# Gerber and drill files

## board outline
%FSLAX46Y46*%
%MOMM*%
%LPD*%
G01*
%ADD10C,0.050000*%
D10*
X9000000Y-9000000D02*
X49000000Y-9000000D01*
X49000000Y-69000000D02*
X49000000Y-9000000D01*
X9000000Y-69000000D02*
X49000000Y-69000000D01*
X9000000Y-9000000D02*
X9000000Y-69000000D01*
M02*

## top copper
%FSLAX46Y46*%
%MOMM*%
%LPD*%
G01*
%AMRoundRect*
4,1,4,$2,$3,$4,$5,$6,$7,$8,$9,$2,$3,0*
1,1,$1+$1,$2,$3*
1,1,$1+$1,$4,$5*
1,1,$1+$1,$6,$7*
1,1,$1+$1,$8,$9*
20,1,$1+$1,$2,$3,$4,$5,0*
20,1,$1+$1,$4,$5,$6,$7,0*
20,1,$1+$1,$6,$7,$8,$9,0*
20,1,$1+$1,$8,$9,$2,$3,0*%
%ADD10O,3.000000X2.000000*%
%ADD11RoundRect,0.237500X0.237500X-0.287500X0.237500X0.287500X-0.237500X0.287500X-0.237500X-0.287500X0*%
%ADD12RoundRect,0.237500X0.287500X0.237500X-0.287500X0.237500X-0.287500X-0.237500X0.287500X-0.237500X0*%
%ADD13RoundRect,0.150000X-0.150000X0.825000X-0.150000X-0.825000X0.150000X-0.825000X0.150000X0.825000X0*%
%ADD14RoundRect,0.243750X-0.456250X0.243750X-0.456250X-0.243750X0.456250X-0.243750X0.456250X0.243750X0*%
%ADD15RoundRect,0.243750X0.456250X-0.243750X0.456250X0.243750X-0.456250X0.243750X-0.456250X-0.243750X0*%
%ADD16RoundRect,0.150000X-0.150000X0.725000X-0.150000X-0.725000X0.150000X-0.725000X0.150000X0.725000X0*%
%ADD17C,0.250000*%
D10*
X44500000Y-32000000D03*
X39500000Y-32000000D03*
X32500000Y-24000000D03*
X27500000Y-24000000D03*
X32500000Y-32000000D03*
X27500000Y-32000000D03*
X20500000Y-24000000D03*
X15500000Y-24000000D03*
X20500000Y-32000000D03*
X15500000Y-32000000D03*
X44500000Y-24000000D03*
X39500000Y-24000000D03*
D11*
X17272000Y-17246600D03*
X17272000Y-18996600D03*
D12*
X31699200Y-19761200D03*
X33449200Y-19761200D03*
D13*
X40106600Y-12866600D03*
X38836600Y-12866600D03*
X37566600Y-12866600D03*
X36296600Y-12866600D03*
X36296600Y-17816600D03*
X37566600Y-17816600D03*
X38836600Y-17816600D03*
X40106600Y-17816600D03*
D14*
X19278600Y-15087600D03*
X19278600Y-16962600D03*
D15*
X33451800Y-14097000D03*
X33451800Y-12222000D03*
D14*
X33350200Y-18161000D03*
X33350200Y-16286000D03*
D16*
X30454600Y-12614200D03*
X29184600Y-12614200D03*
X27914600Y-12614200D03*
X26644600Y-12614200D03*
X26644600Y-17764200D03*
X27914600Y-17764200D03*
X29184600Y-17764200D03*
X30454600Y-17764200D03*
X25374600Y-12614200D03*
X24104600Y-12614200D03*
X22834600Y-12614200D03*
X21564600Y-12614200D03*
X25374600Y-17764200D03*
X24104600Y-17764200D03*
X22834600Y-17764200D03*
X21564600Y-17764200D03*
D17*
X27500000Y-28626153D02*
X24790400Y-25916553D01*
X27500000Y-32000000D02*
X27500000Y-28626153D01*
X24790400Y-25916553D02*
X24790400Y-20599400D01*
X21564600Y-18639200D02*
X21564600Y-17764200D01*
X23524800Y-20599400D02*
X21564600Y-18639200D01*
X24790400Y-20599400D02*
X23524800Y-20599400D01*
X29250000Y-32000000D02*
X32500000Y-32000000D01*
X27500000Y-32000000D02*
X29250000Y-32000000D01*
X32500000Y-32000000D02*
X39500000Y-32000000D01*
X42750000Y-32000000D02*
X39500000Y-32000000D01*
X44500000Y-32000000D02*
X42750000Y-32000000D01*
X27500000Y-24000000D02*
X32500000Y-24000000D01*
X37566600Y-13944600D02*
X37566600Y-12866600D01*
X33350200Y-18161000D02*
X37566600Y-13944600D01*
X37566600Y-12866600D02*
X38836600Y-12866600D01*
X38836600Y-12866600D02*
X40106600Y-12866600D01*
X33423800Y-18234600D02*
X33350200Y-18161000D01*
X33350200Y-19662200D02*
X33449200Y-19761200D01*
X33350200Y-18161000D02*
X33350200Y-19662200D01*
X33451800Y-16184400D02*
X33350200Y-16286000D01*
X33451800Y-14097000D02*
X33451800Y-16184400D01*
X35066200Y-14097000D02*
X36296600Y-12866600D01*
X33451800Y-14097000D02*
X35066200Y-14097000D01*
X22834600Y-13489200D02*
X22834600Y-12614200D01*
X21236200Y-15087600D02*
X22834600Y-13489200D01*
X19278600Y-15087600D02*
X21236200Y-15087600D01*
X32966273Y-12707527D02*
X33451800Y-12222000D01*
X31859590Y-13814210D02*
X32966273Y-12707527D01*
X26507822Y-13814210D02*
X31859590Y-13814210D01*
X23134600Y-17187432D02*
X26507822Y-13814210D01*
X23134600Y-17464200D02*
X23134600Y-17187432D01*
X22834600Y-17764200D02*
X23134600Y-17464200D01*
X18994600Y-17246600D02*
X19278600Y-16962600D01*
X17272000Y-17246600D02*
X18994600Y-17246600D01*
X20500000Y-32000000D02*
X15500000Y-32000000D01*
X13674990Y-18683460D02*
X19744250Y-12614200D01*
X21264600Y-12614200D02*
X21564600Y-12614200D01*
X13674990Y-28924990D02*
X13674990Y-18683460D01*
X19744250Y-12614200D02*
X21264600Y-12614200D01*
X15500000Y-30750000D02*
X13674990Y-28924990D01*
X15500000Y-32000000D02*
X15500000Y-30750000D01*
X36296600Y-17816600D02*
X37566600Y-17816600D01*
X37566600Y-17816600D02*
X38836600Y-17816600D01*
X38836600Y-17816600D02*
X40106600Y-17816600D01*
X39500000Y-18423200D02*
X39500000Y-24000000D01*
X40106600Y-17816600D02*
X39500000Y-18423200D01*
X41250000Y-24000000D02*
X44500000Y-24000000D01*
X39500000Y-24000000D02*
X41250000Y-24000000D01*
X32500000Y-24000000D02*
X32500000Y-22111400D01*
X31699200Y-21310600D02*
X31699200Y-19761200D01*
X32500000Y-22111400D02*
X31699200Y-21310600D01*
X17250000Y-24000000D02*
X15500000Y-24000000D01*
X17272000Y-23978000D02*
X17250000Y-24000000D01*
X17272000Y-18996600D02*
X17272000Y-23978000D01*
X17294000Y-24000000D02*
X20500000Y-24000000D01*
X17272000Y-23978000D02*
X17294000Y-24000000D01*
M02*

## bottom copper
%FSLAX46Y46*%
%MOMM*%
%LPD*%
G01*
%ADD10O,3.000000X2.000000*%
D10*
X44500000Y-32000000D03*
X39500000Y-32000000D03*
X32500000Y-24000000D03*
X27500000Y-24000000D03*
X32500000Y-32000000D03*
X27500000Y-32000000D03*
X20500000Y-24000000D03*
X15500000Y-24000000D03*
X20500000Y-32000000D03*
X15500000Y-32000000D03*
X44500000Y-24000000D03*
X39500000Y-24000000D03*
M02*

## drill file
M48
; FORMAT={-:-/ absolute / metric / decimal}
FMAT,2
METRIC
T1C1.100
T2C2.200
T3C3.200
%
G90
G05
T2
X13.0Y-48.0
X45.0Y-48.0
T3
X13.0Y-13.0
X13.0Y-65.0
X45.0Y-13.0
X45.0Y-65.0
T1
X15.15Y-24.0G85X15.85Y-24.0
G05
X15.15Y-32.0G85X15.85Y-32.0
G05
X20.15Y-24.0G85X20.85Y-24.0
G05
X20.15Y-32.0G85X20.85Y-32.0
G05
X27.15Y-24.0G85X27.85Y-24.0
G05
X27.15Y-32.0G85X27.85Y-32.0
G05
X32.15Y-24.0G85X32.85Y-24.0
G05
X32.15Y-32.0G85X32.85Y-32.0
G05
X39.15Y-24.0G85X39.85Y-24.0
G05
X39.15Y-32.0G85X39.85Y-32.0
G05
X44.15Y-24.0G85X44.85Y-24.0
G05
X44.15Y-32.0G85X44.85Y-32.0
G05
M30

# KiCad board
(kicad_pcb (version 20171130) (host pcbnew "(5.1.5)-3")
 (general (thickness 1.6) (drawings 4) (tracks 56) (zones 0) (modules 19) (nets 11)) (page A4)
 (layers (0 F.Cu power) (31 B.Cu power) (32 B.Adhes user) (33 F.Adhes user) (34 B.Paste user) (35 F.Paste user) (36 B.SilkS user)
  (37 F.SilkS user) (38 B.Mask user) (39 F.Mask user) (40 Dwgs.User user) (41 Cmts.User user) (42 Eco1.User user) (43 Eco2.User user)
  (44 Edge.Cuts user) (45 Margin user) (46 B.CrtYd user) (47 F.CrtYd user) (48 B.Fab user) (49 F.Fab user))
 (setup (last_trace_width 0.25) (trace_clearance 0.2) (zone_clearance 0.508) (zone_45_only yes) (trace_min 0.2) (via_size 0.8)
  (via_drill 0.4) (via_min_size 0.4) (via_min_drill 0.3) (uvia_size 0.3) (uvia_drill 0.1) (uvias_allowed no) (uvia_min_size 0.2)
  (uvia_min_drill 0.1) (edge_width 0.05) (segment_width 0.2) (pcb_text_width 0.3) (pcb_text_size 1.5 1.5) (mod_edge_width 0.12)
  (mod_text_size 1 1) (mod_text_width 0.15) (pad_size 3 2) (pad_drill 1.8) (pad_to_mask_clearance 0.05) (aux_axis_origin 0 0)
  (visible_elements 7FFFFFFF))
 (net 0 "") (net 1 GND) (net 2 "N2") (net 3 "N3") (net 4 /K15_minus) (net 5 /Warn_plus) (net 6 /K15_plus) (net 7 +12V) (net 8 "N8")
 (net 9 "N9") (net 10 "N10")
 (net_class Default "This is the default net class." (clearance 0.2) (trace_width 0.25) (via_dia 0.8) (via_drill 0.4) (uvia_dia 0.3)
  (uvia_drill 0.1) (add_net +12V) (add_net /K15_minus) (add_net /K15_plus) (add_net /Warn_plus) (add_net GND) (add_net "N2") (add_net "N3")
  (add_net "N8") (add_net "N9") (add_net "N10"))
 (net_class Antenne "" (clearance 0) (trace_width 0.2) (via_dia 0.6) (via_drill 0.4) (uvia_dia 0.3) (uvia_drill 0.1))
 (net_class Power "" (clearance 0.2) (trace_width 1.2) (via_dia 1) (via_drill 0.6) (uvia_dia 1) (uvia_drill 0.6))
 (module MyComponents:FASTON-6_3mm (layer F.Cu) (at 42 32)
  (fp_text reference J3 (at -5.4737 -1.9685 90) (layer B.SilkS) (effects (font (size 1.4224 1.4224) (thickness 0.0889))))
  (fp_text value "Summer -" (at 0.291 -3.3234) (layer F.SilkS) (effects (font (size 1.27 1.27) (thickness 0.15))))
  (pad 1 thru_hole oval (at 2.5 0) (size 3 2) (drill oval 1.8 1.1) (layers *.Cu *.Paste *.Mask F.SilkS) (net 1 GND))
  (pad 1 thru_hole oval (at -2.5 0) (size 3 2) (drill oval 1.8 1.1) (layers *.Cu *.Paste *.Mask F.SilkS) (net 1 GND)))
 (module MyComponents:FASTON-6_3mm (layer F.Cu) (at 30 24)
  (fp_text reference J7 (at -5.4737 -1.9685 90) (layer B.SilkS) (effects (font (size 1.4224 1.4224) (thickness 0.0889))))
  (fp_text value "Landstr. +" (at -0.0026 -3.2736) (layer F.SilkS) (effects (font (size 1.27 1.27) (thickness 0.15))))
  (pad 1 thru_hole oval (at 2.5 0) (size 3 2) (drill oval 1.8 1.1) (layers *.Cu *.Paste *.Mask F.SilkS) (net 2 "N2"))
  (pad 1 thru_hole oval (at -2.5 0) (size 3 2) (drill oval 1.8 1.1) (layers *.Cu *.Paste *.Mask F.SilkS) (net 2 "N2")))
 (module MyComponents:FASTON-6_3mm (layer F.Cu) (at 30 32)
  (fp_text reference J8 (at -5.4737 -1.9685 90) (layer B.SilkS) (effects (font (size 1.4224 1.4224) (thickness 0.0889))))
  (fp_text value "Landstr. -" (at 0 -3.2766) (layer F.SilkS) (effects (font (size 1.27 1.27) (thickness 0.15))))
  (pad 1 thru_hole oval (at 2.5 0) (size 3 2) (drill oval 1.8 1.1) (layers *.Cu *.Paste *.Mask F.SilkS) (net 1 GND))
  (pad 1 thru_hole oval (at -2.5 0) (size 3 2) (drill oval 1.8 1.1) (layers *.Cu *.Paste *.Mask F.SilkS) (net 1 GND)))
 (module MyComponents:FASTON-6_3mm (layer F.Cu) (at 18 24)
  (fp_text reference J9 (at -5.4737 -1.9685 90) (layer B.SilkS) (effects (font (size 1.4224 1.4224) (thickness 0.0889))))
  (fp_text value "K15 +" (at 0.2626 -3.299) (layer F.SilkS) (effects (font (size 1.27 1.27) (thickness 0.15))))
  (pad 1 thru_hole oval (at 2.5 0) (size 3 2) (drill oval 1.8 1.1) (layers *.Cu *.Paste *.Mask F.SilkS) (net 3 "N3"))
  (pad 1 thru_hole oval (at -2.5 0) (size 3 2) (drill oval 1.8 1.1) (layers *.Cu *.Paste *.Mask F.SilkS) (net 3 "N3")))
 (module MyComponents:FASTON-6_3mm (layer F.Cu) (at 18 32)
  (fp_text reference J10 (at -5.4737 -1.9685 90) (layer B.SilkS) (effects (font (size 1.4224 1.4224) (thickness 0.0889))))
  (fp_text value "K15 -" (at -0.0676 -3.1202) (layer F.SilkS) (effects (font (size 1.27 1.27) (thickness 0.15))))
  (pad 1 thru_hole oval (at 2.5 0) (size 3 2) (drill oval 1.8 1.1) (layers *.Cu *.Paste *.Mask F.SilkS) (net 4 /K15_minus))
  (pad 1 thru_hole oval (at -2.5 0) (size 3 2) (drill oval 1.8 1.1) (layers *.Cu *.Paste *.Mask F.SilkS) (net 4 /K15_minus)))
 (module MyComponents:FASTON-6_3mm (layer F.Cu) (at 42 24)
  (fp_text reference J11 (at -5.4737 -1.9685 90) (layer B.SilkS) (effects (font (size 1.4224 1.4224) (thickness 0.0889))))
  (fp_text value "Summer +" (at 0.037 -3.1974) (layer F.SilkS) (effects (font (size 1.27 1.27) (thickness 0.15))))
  (pad 1 thru_hole oval (at 2.5 0) (size 3 2) (drill oval 1.8 1.1) (layers *.Cu *.Paste *.Mask F.SilkS) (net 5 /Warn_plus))
  (pad 1 thru_hole oval (at -2.5 0) (size 3 2) (drill oval 1.8 1.1) (layers *.Cu *.Paste *.Mask F.SilkS) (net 5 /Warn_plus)))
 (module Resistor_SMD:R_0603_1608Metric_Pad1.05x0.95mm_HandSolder (layer F.Cu) (at 17.272 18.1216 90)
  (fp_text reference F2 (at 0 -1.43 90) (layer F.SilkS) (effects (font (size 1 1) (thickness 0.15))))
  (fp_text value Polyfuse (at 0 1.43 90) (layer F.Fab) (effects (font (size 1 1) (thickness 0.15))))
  (pad 2 smd roundrect (at 0.875 0 90) (size 1.05 0.95) (layers F.Cu F.Paste F.Mask) (roundrect_rratio 0.25) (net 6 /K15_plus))
  (pad 1 smd roundrect (at -0.875 0 90) (size 1.05 0.95) (layers F.Cu F.Paste F.Mask) (roundrect_rratio 0.25) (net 3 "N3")))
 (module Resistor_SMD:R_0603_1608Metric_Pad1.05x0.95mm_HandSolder (layer F.Cu) (at 32.5742 19.7612 180)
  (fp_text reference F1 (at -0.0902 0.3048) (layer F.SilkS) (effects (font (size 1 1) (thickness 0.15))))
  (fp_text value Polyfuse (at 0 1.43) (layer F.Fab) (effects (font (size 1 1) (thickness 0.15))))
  (pad 2 smd roundrect (at 0.875 0 180) (size 1.05 0.95) (layers F.Cu F.Paste F.Mask) (roundrect_rratio 0.25) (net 2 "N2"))
  (pad 1 smd roundrect (at -0.875 0 180) (size 1.05 0.95) (layers F.Cu F.Paste F.Mask) (roundrect_rratio 0.25) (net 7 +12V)))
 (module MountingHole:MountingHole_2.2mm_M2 (layer F.Cu) (at 45 48)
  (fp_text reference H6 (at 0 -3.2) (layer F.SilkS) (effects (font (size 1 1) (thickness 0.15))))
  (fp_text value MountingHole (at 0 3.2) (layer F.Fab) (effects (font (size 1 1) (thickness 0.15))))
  (pad 1 np_thru_hole circle (at 0 0) (size 2.2 2.2) (drill 2.2) (layers *.Cu *.Mask)))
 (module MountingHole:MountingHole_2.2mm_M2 (layer F.Cu) (at 13 48)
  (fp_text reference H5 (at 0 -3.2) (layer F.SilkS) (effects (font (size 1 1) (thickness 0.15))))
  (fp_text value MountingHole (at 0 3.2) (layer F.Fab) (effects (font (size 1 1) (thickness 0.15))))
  (pad 1 np_thru_hole circle (at 0 0) (size 2.2 2.2) (drill 2.2) (layers *.Cu *.Mask)))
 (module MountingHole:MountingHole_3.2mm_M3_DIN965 (layer F.Cu) (at 13 13)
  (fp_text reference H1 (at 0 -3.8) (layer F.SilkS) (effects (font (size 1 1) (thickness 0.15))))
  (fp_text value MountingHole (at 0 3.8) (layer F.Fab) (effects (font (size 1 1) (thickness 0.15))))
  (pad 1 np_thru_hole circle (at 0 0) (size 3.2 3.2) (drill 3.2) (layers *.Cu *.Mask)))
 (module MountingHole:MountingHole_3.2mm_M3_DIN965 (layer F.Cu) (at 13 65)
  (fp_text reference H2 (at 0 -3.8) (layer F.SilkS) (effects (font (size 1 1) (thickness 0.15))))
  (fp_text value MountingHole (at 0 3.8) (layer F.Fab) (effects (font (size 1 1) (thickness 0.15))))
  (pad 1 np_thru_hole circle (at 0 0) (size 3.2 3.2) (drill 3.2) (layers *.Cu *.Mask)))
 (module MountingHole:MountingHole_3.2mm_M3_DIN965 (layer F.Cu) (at 45 13)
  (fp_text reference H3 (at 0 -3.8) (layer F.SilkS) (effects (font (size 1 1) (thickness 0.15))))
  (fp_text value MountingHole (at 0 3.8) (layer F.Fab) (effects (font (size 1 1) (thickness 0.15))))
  (pad 1 np_thru_hole circle (at 0 0) (size 3.2 3.2) (drill 3.2) (layers *.Cu *.Mask)))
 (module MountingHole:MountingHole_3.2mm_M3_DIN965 (layer F.Cu) (at 45 65)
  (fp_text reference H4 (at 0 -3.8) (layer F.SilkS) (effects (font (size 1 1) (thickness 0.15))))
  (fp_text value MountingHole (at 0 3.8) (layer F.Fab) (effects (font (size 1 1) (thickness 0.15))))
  (pad 1 np_thru_hole circle (at 0 0) (size 3.2 3.2) (drill 3.2) (layers *.Cu *.Mask)))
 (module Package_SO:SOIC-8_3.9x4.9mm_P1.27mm (layer F.Cu) (at 38.2016 15.3416 270)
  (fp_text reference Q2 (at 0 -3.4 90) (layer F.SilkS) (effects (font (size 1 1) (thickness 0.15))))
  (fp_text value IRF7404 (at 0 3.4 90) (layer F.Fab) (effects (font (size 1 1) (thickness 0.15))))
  (pad 1 smd roundrect (at -2.475 -1.905 270) (size 1.95 0.6) (layers F.Cu F.Paste F.Mask) (roundrect_rratio 0.25) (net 7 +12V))
  (pad 2 smd roundrect (at -2.475 -0.635 270) (size 1.95 0.6) (layers F.Cu F.Paste F.Mask) (roundrect_rratio 0.25) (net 7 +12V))
  (pad 3 smd roundrect (at -2.475 0.635 270) (size 1.95 0.6) (layers F.Cu F.Paste F.Mask) (roundrect_rratio 0.25) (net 7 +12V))
  (pad 4 smd roundrect (at -2.475 1.905 270) (size 1.95 0.6) (layers F.Cu F.Paste F.Mask) (roundrect_rratio 0.25) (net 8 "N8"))
  (pad 5 smd roundrect (at 2.475 1.905 270) (size 1.95 0.6) (layers F.Cu F.Paste F.Mask) (roundrect_rratio 0.25) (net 5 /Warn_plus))
  (pad 6 smd roundrect (at 2.475 0.635 270) (size 1.95 0.6) (layers F.Cu F.Paste F.Mask) (roundrect_rratio 0.25) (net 5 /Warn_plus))
  (pad 7 smd roundrect (at 2.475 -0.635 270) (size 1.95 0.6) (layers F.Cu F.Paste F.Mask) (roundrect_rratio 0.25) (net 5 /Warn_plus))
  (pad 8 smd roundrect (at 2.475 -1.905 270) (size 1.95 0.6) (layers F.Cu F.Paste F.Mask) (roundrect_rratio 0.25) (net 5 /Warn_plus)))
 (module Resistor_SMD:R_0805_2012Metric (layer F.Cu) (at 19.2786 16.0251 270)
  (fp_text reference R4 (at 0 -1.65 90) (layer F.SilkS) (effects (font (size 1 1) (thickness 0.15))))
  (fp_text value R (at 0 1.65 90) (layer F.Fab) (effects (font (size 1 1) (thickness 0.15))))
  (pad 1 smd roundrect (at -0.9375 0 270) (size 0.975 1.4) (layers F.Cu F.Paste F.Mask) (roundrect_rratio 0.25) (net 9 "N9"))
  (pad 2 smd roundrect (at 0.9375 0 270) (size 0.975 1.4) (layers F.Cu F.Paste F.Mask) (roundrect_rratio 0.25) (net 6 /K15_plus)))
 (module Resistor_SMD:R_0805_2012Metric (layer F.Cu) (at 33.4518 13.1595 90)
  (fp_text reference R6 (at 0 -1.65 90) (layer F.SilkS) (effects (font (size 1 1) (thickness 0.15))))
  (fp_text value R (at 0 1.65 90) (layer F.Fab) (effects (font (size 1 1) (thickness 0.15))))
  (pad 1 smd roundrect (at -0.9375 0 90) (size 0.975 1.4) (layers F.Cu F.Paste F.Mask) (roundrect_rratio 0.25) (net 8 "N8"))
  (pad 2 smd roundrect (at 0.9375 0 90) (size 0.975 1.4) (layers F.Cu F.Paste F.Mask) (roundrect_rratio 0.25) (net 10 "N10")))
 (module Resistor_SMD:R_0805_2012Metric (layer F.Cu) (at 33.3502 17.2235 270)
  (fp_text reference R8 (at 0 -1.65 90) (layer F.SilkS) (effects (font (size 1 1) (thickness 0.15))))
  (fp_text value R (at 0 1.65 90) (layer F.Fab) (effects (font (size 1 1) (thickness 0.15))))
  (pad 2 smd roundrect (at 0.9375 0 270) (size 0.975 1.4) (layers F.Cu F.Paste F.Mask) (roundrect_rratio 0.25) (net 7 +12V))
  (pad 1 smd roundrect (at -0.9375 0 270) (size 0.975 1.4) (layers F.Cu F.Paste F.Mask) (roundrect_rratio 0.25) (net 8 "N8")))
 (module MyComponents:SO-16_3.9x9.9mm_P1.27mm (layer F.Cu) (at 28.5496 15.1892 270)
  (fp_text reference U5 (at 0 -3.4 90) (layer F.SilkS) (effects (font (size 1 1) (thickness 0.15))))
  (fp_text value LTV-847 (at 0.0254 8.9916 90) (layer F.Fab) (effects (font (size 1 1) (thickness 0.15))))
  (pad 1 smd roundrect (at -2.575 -1.905 270) (size 1.75 0.6) (layers F.Cu F.Paste F.Mask) (roundrect_rratio 0.25))
  (pad 2 smd roundrect (at -2.575 -0.635 270) (size 1.75 0.6) (layers F.Cu F.Paste F.Mask) (roundrect_rratio 0.25))
  (pad 3 smd roundrect (at -2.575 0.635 270) (size 1.75 0.6) (layers F.Cu F.Paste F.Mask) (roundrect_rratio 0.25))
  (pad 4 smd roundrect (at -2.575 1.905 270) (size 1.75 0.6) (layers F.Cu F.Paste F.Mask) (roundrect_rratio 0.25))
  (pad 13 smd roundrect (at 2.575 1.905 270) (size 1.75 0.6) (layers F.Cu F.Paste F.Mask) (roundrect_rratio 0.25))
  (pad 14 smd roundrect (at 2.575 0.635 270) (size 1.75 0.6) (layers F.Cu F.Paste F.Mask) (roundrect_rratio 0.25))
  (pad 15 smd roundrect (at 2.575 -0.635 270) (size 1.75 0.6) (layers F.Cu F.Paste F.Mask) (roundrect_rratio 0.25))
  (pad 16 smd roundrect (at 2.575 -1.905 270) (size 1.75 0.6) (layers F.Cu F.Paste F.Mask) (roundrect_rratio 0.25))
  (pad 5 smd roundrect (at -2.575 3.175 270) (size 1.75 0.6) (layers F.Cu F.Paste F.Mask) (roundrect_rratio 0.25))
  (pad 6 smd roundrect (at -2.575 4.445 270) (size 1.75 0.6) (layers F.Cu F.Paste F.Mask) (roundrect_rratio 0.25))
  (pad 7 smd roundrect (at -2.575 5.715 270) (size 1.75 0.6) (layers F.Cu F.Paste F.Mask) (roundrect_rratio 0.25) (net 9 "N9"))
  (pad 8 smd roundrect (at -2.575 6.985 270) (size 1.75 0.6) (layers F.Cu F.Paste F.Mask) (roundrect_rratio 0.25) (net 4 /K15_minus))
  (pad 12 smd roundrect (at 2.575 3.175 270) (size 1.75 0.6) (layers F.Cu F.Paste F.Mask) (roundrect_rratio 0.25))
  (pad 11 smd roundrect (at 2.575 4.445 270) (size 1.75 0.6) (layers F.Cu F.Paste F.Mask) (roundrect_rratio 0.25))
  (pad 10 smd roundrect (at 2.575 5.715 270) (size 1.75 0.6) (layers F.Cu F.Paste F.Mask) (roundrect_rratio 0.25) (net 10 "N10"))
  (pad 9 smd roundrect (at 2.575 6.985 270) (size 1.75 0.6) (layers F.Cu F.Paste F.Mask) (roundrect_rratio 0.25) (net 1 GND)))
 (gr_line (start 9 9) (end 49 9) (layer Edge.Cuts) (width 0.05))
 (gr_line (start 49 69) (end 49 9) (layer Edge.Cuts) (width 0.05))
 (gr_line (start 9 69) (end 49 69) (layer Edge.Cuts) (width 0.05))
 (gr_line (start 9 9) (end 9 69) (layer Edge.Cuts) (width 0.05))
 (segment (start 27.5 28.626153) (end 24.7904 25.916553) (width 0.25) (layer F.Cu) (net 1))
 (segment (start 27.5 32) (end 27.5 28.626153) (width 0.25) (layer F.Cu) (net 1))
 (segment (start 24.7904 25.916553) (end 24.7904 20.5994) (width 0.25) (layer F.Cu) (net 1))
 (segment (start 21.5646 18.6392) (end 21.5646 17.7642) (width 0.25) (layer F.Cu) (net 1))
 (segment (start 23.5248 20.5994) (end 21.5646 18.6392) (width 0.25) (layer F.Cu) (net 1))
 (segment (start 24.7904 20.5994) (end 23.5248 20.5994) (width 0.25) (layer F.Cu) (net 1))
 (segment (start 29.25 32) (end 32.5 32) (width 0.25) (layer F.Cu) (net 1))
 (segment (start 27.5 32) (end 29.25 32) (width 0.25) (layer F.Cu) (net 1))
 (segment (start 32.5 32) (end 39.5 32) (width 0.25) (layer F.Cu) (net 1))
 (segment (start 42.75 32) (end 39.5 32) (width 0.25) (layer F.Cu) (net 1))
 (segment (start 44.5 32) (end 42.75 32) (width 0.25) (layer F.Cu) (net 1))
 (segment (start 27.5 24) (end 32.5 24) (width 0.25) (layer F.Cu) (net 2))
 (segment (start 37.5666 13.9446) (end 37.5666 12.8666) (width 0.25) (layer F.Cu) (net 7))
 (segment (start 33.3502 18.161) (end 37.5666 13.9446) (width 0.25) (layer F.Cu) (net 7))
 (segment (start 37.5666 12.8666) (end 38.8366 12.8666) (width 0.25) (layer F.Cu) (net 7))
 (segment (start 38.8366 12.8666) (end 40.1066 12.8666) (width 0.25) (layer F.Cu) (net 7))
 (segment (start 33.4238 18.2346) (end 33.3502 18.161) (width 0.25) (layer F.Cu) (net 7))
 (segment (start 33.3502 19.6622) (end 33.4492 19.7612) (width 0.25) (layer F.Cu) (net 7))
 (segment (start 33.3502 18.161) (end 33.3502 19.6622) (width 0.25) (layer F.Cu) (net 7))
 (segment (start 33.4518 16.1844) (end 33.3502 16.286) (width 0.25) (layer F.Cu) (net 8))
 (segment (start 33.4518 14.097) (end 33.4518 16.1844) (width 0.25) (layer F.Cu) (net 8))
 (segment (start 35.0662 14.097) (end 36.2966 12.8666) (width 0.25) (layer F.Cu) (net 8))
 (segment (start 33.4518 14.097) (end 35.0662 14.097) (width 0.25) (layer F.Cu) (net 8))
 (segment (start 22.8346 13.4892) (end 22.8346 12.6142) (width 0.25) (layer F.Cu) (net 9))
 (segment (start 21.2362 15.0876) (end 22.8346 13.4892) (width 0.25) (layer F.Cu) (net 9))
 (segment (start 19.2786 15.0876) (end 21.2362 15.0876) (width 0.25) (layer F.Cu) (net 9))
 (segment (start 32.966273 12.707527) (end 33.4518 12.222) (width 0.25) (layer F.Cu) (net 10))
 (segment (start 31.85959 13.81421) (end 32.966273 12.707527) (width 0.25) (layer F.Cu) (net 10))
 (segment (start 26.507822 13.81421) (end 31.85959 13.81421) (width 0.25) (layer F.Cu) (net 10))
 (segment (start 23.1346 17.187432) (end 26.507822 13.81421) (width 0.25) (layer F.Cu) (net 10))
 (segment (start 23.1346 17.4642) (end 23.1346 17.187432) (width 0.25) (layer F.Cu) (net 10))
 (segment (start 22.8346 17.7642) (end 23.1346 17.4642) (width 0.25) (layer F.Cu) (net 10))
 (segment (start 18.9946 17.2466) (end 19.2786 16.9626) (width 0.25) (layer F.Cu) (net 6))
 (segment (start 17.272 17.2466) (end 18.9946 17.2466) (width 0.25) (layer F.Cu) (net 6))
 (segment (start 20.5 32) (end 15.5 32) (width 0.25) (layer F.Cu) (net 4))
 (segment (start 13.67499 18.68346) (end 19.74425 12.6142) (width 0.25) (layer F.Cu) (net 4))
 (segment (start 21.2646 12.6142) (end 21.5646 12.6142) (width 0.25) (layer F.Cu) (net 4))
 (segment (start 13.67499 28.92499) (end 13.67499 18.68346) (width 0.25) (layer F.Cu) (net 4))
 (segment (start 19.74425 12.6142) (end 21.2646 12.6142) (width 0.25) (layer F.Cu) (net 4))
 (segment (start 15.5 30.75) (end 13.67499 28.92499) (width 0.25) (layer F.Cu) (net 4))
 (segment (start 15.5 32) (end 15.5 30.75) (width 0.25) (layer F.Cu) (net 4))
 (segment (start 36.2966 17.8166) (end 37.5666 17.8166) (width 0.25) (layer F.Cu) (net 5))
 (segment (start 37.5666 17.8166) (end 38.8366 17.8166) (width 0.25) (layer F.Cu) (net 5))
 (segment (start 38.8366 17.8166) (end 40.1066 17.8166) (width 0.25) (layer F.Cu) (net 5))
 (segment (start 39.5 18.4232) (end 39.5 24) (width 0.25) (layer F.Cu) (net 5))
 (segment (start 40.1066 17.8166) (end 39.5 18.4232) (width 0.25) (layer F.Cu) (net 5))
 (segment (start 41.25 24) (end 44.5 24) (width 0.25) (layer F.Cu) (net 5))
 (segment (start 39.5 24) (end 41.25 24) (width 0.25) (layer F.Cu) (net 5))
 (segment (start 32.5 24) (end 32.5 22.1114) (width 0.25) (layer F.Cu) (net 2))
 (segment (start 31.6992 21.3106) (end 31.6992 19.7612) (width 0.25) (layer F.Cu) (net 2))
 (segment (start 32.5 22.1114) (end 31.6992 21.3106) (width 0.25) (layer F.Cu) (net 2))
 (segment (start 17.25 24) (end 15.5 24) (width 0.25) (layer F.Cu) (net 3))
 (segment (start 17.272 23.978) (end 17.25 24) (width 0.25) (layer F.Cu) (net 3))
 (segment (start 17.272 18.9966) (end 17.272 23.978) (width 0.25) (layer F.Cu) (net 3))
 (segment (start 17.294 24) (end 20.5 24) (width 0.25) (layer F.Cu) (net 3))
 (segment (start 17.272 23.978) (end 17.294 24) (width 0.25) (layer F.Cu) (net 3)))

